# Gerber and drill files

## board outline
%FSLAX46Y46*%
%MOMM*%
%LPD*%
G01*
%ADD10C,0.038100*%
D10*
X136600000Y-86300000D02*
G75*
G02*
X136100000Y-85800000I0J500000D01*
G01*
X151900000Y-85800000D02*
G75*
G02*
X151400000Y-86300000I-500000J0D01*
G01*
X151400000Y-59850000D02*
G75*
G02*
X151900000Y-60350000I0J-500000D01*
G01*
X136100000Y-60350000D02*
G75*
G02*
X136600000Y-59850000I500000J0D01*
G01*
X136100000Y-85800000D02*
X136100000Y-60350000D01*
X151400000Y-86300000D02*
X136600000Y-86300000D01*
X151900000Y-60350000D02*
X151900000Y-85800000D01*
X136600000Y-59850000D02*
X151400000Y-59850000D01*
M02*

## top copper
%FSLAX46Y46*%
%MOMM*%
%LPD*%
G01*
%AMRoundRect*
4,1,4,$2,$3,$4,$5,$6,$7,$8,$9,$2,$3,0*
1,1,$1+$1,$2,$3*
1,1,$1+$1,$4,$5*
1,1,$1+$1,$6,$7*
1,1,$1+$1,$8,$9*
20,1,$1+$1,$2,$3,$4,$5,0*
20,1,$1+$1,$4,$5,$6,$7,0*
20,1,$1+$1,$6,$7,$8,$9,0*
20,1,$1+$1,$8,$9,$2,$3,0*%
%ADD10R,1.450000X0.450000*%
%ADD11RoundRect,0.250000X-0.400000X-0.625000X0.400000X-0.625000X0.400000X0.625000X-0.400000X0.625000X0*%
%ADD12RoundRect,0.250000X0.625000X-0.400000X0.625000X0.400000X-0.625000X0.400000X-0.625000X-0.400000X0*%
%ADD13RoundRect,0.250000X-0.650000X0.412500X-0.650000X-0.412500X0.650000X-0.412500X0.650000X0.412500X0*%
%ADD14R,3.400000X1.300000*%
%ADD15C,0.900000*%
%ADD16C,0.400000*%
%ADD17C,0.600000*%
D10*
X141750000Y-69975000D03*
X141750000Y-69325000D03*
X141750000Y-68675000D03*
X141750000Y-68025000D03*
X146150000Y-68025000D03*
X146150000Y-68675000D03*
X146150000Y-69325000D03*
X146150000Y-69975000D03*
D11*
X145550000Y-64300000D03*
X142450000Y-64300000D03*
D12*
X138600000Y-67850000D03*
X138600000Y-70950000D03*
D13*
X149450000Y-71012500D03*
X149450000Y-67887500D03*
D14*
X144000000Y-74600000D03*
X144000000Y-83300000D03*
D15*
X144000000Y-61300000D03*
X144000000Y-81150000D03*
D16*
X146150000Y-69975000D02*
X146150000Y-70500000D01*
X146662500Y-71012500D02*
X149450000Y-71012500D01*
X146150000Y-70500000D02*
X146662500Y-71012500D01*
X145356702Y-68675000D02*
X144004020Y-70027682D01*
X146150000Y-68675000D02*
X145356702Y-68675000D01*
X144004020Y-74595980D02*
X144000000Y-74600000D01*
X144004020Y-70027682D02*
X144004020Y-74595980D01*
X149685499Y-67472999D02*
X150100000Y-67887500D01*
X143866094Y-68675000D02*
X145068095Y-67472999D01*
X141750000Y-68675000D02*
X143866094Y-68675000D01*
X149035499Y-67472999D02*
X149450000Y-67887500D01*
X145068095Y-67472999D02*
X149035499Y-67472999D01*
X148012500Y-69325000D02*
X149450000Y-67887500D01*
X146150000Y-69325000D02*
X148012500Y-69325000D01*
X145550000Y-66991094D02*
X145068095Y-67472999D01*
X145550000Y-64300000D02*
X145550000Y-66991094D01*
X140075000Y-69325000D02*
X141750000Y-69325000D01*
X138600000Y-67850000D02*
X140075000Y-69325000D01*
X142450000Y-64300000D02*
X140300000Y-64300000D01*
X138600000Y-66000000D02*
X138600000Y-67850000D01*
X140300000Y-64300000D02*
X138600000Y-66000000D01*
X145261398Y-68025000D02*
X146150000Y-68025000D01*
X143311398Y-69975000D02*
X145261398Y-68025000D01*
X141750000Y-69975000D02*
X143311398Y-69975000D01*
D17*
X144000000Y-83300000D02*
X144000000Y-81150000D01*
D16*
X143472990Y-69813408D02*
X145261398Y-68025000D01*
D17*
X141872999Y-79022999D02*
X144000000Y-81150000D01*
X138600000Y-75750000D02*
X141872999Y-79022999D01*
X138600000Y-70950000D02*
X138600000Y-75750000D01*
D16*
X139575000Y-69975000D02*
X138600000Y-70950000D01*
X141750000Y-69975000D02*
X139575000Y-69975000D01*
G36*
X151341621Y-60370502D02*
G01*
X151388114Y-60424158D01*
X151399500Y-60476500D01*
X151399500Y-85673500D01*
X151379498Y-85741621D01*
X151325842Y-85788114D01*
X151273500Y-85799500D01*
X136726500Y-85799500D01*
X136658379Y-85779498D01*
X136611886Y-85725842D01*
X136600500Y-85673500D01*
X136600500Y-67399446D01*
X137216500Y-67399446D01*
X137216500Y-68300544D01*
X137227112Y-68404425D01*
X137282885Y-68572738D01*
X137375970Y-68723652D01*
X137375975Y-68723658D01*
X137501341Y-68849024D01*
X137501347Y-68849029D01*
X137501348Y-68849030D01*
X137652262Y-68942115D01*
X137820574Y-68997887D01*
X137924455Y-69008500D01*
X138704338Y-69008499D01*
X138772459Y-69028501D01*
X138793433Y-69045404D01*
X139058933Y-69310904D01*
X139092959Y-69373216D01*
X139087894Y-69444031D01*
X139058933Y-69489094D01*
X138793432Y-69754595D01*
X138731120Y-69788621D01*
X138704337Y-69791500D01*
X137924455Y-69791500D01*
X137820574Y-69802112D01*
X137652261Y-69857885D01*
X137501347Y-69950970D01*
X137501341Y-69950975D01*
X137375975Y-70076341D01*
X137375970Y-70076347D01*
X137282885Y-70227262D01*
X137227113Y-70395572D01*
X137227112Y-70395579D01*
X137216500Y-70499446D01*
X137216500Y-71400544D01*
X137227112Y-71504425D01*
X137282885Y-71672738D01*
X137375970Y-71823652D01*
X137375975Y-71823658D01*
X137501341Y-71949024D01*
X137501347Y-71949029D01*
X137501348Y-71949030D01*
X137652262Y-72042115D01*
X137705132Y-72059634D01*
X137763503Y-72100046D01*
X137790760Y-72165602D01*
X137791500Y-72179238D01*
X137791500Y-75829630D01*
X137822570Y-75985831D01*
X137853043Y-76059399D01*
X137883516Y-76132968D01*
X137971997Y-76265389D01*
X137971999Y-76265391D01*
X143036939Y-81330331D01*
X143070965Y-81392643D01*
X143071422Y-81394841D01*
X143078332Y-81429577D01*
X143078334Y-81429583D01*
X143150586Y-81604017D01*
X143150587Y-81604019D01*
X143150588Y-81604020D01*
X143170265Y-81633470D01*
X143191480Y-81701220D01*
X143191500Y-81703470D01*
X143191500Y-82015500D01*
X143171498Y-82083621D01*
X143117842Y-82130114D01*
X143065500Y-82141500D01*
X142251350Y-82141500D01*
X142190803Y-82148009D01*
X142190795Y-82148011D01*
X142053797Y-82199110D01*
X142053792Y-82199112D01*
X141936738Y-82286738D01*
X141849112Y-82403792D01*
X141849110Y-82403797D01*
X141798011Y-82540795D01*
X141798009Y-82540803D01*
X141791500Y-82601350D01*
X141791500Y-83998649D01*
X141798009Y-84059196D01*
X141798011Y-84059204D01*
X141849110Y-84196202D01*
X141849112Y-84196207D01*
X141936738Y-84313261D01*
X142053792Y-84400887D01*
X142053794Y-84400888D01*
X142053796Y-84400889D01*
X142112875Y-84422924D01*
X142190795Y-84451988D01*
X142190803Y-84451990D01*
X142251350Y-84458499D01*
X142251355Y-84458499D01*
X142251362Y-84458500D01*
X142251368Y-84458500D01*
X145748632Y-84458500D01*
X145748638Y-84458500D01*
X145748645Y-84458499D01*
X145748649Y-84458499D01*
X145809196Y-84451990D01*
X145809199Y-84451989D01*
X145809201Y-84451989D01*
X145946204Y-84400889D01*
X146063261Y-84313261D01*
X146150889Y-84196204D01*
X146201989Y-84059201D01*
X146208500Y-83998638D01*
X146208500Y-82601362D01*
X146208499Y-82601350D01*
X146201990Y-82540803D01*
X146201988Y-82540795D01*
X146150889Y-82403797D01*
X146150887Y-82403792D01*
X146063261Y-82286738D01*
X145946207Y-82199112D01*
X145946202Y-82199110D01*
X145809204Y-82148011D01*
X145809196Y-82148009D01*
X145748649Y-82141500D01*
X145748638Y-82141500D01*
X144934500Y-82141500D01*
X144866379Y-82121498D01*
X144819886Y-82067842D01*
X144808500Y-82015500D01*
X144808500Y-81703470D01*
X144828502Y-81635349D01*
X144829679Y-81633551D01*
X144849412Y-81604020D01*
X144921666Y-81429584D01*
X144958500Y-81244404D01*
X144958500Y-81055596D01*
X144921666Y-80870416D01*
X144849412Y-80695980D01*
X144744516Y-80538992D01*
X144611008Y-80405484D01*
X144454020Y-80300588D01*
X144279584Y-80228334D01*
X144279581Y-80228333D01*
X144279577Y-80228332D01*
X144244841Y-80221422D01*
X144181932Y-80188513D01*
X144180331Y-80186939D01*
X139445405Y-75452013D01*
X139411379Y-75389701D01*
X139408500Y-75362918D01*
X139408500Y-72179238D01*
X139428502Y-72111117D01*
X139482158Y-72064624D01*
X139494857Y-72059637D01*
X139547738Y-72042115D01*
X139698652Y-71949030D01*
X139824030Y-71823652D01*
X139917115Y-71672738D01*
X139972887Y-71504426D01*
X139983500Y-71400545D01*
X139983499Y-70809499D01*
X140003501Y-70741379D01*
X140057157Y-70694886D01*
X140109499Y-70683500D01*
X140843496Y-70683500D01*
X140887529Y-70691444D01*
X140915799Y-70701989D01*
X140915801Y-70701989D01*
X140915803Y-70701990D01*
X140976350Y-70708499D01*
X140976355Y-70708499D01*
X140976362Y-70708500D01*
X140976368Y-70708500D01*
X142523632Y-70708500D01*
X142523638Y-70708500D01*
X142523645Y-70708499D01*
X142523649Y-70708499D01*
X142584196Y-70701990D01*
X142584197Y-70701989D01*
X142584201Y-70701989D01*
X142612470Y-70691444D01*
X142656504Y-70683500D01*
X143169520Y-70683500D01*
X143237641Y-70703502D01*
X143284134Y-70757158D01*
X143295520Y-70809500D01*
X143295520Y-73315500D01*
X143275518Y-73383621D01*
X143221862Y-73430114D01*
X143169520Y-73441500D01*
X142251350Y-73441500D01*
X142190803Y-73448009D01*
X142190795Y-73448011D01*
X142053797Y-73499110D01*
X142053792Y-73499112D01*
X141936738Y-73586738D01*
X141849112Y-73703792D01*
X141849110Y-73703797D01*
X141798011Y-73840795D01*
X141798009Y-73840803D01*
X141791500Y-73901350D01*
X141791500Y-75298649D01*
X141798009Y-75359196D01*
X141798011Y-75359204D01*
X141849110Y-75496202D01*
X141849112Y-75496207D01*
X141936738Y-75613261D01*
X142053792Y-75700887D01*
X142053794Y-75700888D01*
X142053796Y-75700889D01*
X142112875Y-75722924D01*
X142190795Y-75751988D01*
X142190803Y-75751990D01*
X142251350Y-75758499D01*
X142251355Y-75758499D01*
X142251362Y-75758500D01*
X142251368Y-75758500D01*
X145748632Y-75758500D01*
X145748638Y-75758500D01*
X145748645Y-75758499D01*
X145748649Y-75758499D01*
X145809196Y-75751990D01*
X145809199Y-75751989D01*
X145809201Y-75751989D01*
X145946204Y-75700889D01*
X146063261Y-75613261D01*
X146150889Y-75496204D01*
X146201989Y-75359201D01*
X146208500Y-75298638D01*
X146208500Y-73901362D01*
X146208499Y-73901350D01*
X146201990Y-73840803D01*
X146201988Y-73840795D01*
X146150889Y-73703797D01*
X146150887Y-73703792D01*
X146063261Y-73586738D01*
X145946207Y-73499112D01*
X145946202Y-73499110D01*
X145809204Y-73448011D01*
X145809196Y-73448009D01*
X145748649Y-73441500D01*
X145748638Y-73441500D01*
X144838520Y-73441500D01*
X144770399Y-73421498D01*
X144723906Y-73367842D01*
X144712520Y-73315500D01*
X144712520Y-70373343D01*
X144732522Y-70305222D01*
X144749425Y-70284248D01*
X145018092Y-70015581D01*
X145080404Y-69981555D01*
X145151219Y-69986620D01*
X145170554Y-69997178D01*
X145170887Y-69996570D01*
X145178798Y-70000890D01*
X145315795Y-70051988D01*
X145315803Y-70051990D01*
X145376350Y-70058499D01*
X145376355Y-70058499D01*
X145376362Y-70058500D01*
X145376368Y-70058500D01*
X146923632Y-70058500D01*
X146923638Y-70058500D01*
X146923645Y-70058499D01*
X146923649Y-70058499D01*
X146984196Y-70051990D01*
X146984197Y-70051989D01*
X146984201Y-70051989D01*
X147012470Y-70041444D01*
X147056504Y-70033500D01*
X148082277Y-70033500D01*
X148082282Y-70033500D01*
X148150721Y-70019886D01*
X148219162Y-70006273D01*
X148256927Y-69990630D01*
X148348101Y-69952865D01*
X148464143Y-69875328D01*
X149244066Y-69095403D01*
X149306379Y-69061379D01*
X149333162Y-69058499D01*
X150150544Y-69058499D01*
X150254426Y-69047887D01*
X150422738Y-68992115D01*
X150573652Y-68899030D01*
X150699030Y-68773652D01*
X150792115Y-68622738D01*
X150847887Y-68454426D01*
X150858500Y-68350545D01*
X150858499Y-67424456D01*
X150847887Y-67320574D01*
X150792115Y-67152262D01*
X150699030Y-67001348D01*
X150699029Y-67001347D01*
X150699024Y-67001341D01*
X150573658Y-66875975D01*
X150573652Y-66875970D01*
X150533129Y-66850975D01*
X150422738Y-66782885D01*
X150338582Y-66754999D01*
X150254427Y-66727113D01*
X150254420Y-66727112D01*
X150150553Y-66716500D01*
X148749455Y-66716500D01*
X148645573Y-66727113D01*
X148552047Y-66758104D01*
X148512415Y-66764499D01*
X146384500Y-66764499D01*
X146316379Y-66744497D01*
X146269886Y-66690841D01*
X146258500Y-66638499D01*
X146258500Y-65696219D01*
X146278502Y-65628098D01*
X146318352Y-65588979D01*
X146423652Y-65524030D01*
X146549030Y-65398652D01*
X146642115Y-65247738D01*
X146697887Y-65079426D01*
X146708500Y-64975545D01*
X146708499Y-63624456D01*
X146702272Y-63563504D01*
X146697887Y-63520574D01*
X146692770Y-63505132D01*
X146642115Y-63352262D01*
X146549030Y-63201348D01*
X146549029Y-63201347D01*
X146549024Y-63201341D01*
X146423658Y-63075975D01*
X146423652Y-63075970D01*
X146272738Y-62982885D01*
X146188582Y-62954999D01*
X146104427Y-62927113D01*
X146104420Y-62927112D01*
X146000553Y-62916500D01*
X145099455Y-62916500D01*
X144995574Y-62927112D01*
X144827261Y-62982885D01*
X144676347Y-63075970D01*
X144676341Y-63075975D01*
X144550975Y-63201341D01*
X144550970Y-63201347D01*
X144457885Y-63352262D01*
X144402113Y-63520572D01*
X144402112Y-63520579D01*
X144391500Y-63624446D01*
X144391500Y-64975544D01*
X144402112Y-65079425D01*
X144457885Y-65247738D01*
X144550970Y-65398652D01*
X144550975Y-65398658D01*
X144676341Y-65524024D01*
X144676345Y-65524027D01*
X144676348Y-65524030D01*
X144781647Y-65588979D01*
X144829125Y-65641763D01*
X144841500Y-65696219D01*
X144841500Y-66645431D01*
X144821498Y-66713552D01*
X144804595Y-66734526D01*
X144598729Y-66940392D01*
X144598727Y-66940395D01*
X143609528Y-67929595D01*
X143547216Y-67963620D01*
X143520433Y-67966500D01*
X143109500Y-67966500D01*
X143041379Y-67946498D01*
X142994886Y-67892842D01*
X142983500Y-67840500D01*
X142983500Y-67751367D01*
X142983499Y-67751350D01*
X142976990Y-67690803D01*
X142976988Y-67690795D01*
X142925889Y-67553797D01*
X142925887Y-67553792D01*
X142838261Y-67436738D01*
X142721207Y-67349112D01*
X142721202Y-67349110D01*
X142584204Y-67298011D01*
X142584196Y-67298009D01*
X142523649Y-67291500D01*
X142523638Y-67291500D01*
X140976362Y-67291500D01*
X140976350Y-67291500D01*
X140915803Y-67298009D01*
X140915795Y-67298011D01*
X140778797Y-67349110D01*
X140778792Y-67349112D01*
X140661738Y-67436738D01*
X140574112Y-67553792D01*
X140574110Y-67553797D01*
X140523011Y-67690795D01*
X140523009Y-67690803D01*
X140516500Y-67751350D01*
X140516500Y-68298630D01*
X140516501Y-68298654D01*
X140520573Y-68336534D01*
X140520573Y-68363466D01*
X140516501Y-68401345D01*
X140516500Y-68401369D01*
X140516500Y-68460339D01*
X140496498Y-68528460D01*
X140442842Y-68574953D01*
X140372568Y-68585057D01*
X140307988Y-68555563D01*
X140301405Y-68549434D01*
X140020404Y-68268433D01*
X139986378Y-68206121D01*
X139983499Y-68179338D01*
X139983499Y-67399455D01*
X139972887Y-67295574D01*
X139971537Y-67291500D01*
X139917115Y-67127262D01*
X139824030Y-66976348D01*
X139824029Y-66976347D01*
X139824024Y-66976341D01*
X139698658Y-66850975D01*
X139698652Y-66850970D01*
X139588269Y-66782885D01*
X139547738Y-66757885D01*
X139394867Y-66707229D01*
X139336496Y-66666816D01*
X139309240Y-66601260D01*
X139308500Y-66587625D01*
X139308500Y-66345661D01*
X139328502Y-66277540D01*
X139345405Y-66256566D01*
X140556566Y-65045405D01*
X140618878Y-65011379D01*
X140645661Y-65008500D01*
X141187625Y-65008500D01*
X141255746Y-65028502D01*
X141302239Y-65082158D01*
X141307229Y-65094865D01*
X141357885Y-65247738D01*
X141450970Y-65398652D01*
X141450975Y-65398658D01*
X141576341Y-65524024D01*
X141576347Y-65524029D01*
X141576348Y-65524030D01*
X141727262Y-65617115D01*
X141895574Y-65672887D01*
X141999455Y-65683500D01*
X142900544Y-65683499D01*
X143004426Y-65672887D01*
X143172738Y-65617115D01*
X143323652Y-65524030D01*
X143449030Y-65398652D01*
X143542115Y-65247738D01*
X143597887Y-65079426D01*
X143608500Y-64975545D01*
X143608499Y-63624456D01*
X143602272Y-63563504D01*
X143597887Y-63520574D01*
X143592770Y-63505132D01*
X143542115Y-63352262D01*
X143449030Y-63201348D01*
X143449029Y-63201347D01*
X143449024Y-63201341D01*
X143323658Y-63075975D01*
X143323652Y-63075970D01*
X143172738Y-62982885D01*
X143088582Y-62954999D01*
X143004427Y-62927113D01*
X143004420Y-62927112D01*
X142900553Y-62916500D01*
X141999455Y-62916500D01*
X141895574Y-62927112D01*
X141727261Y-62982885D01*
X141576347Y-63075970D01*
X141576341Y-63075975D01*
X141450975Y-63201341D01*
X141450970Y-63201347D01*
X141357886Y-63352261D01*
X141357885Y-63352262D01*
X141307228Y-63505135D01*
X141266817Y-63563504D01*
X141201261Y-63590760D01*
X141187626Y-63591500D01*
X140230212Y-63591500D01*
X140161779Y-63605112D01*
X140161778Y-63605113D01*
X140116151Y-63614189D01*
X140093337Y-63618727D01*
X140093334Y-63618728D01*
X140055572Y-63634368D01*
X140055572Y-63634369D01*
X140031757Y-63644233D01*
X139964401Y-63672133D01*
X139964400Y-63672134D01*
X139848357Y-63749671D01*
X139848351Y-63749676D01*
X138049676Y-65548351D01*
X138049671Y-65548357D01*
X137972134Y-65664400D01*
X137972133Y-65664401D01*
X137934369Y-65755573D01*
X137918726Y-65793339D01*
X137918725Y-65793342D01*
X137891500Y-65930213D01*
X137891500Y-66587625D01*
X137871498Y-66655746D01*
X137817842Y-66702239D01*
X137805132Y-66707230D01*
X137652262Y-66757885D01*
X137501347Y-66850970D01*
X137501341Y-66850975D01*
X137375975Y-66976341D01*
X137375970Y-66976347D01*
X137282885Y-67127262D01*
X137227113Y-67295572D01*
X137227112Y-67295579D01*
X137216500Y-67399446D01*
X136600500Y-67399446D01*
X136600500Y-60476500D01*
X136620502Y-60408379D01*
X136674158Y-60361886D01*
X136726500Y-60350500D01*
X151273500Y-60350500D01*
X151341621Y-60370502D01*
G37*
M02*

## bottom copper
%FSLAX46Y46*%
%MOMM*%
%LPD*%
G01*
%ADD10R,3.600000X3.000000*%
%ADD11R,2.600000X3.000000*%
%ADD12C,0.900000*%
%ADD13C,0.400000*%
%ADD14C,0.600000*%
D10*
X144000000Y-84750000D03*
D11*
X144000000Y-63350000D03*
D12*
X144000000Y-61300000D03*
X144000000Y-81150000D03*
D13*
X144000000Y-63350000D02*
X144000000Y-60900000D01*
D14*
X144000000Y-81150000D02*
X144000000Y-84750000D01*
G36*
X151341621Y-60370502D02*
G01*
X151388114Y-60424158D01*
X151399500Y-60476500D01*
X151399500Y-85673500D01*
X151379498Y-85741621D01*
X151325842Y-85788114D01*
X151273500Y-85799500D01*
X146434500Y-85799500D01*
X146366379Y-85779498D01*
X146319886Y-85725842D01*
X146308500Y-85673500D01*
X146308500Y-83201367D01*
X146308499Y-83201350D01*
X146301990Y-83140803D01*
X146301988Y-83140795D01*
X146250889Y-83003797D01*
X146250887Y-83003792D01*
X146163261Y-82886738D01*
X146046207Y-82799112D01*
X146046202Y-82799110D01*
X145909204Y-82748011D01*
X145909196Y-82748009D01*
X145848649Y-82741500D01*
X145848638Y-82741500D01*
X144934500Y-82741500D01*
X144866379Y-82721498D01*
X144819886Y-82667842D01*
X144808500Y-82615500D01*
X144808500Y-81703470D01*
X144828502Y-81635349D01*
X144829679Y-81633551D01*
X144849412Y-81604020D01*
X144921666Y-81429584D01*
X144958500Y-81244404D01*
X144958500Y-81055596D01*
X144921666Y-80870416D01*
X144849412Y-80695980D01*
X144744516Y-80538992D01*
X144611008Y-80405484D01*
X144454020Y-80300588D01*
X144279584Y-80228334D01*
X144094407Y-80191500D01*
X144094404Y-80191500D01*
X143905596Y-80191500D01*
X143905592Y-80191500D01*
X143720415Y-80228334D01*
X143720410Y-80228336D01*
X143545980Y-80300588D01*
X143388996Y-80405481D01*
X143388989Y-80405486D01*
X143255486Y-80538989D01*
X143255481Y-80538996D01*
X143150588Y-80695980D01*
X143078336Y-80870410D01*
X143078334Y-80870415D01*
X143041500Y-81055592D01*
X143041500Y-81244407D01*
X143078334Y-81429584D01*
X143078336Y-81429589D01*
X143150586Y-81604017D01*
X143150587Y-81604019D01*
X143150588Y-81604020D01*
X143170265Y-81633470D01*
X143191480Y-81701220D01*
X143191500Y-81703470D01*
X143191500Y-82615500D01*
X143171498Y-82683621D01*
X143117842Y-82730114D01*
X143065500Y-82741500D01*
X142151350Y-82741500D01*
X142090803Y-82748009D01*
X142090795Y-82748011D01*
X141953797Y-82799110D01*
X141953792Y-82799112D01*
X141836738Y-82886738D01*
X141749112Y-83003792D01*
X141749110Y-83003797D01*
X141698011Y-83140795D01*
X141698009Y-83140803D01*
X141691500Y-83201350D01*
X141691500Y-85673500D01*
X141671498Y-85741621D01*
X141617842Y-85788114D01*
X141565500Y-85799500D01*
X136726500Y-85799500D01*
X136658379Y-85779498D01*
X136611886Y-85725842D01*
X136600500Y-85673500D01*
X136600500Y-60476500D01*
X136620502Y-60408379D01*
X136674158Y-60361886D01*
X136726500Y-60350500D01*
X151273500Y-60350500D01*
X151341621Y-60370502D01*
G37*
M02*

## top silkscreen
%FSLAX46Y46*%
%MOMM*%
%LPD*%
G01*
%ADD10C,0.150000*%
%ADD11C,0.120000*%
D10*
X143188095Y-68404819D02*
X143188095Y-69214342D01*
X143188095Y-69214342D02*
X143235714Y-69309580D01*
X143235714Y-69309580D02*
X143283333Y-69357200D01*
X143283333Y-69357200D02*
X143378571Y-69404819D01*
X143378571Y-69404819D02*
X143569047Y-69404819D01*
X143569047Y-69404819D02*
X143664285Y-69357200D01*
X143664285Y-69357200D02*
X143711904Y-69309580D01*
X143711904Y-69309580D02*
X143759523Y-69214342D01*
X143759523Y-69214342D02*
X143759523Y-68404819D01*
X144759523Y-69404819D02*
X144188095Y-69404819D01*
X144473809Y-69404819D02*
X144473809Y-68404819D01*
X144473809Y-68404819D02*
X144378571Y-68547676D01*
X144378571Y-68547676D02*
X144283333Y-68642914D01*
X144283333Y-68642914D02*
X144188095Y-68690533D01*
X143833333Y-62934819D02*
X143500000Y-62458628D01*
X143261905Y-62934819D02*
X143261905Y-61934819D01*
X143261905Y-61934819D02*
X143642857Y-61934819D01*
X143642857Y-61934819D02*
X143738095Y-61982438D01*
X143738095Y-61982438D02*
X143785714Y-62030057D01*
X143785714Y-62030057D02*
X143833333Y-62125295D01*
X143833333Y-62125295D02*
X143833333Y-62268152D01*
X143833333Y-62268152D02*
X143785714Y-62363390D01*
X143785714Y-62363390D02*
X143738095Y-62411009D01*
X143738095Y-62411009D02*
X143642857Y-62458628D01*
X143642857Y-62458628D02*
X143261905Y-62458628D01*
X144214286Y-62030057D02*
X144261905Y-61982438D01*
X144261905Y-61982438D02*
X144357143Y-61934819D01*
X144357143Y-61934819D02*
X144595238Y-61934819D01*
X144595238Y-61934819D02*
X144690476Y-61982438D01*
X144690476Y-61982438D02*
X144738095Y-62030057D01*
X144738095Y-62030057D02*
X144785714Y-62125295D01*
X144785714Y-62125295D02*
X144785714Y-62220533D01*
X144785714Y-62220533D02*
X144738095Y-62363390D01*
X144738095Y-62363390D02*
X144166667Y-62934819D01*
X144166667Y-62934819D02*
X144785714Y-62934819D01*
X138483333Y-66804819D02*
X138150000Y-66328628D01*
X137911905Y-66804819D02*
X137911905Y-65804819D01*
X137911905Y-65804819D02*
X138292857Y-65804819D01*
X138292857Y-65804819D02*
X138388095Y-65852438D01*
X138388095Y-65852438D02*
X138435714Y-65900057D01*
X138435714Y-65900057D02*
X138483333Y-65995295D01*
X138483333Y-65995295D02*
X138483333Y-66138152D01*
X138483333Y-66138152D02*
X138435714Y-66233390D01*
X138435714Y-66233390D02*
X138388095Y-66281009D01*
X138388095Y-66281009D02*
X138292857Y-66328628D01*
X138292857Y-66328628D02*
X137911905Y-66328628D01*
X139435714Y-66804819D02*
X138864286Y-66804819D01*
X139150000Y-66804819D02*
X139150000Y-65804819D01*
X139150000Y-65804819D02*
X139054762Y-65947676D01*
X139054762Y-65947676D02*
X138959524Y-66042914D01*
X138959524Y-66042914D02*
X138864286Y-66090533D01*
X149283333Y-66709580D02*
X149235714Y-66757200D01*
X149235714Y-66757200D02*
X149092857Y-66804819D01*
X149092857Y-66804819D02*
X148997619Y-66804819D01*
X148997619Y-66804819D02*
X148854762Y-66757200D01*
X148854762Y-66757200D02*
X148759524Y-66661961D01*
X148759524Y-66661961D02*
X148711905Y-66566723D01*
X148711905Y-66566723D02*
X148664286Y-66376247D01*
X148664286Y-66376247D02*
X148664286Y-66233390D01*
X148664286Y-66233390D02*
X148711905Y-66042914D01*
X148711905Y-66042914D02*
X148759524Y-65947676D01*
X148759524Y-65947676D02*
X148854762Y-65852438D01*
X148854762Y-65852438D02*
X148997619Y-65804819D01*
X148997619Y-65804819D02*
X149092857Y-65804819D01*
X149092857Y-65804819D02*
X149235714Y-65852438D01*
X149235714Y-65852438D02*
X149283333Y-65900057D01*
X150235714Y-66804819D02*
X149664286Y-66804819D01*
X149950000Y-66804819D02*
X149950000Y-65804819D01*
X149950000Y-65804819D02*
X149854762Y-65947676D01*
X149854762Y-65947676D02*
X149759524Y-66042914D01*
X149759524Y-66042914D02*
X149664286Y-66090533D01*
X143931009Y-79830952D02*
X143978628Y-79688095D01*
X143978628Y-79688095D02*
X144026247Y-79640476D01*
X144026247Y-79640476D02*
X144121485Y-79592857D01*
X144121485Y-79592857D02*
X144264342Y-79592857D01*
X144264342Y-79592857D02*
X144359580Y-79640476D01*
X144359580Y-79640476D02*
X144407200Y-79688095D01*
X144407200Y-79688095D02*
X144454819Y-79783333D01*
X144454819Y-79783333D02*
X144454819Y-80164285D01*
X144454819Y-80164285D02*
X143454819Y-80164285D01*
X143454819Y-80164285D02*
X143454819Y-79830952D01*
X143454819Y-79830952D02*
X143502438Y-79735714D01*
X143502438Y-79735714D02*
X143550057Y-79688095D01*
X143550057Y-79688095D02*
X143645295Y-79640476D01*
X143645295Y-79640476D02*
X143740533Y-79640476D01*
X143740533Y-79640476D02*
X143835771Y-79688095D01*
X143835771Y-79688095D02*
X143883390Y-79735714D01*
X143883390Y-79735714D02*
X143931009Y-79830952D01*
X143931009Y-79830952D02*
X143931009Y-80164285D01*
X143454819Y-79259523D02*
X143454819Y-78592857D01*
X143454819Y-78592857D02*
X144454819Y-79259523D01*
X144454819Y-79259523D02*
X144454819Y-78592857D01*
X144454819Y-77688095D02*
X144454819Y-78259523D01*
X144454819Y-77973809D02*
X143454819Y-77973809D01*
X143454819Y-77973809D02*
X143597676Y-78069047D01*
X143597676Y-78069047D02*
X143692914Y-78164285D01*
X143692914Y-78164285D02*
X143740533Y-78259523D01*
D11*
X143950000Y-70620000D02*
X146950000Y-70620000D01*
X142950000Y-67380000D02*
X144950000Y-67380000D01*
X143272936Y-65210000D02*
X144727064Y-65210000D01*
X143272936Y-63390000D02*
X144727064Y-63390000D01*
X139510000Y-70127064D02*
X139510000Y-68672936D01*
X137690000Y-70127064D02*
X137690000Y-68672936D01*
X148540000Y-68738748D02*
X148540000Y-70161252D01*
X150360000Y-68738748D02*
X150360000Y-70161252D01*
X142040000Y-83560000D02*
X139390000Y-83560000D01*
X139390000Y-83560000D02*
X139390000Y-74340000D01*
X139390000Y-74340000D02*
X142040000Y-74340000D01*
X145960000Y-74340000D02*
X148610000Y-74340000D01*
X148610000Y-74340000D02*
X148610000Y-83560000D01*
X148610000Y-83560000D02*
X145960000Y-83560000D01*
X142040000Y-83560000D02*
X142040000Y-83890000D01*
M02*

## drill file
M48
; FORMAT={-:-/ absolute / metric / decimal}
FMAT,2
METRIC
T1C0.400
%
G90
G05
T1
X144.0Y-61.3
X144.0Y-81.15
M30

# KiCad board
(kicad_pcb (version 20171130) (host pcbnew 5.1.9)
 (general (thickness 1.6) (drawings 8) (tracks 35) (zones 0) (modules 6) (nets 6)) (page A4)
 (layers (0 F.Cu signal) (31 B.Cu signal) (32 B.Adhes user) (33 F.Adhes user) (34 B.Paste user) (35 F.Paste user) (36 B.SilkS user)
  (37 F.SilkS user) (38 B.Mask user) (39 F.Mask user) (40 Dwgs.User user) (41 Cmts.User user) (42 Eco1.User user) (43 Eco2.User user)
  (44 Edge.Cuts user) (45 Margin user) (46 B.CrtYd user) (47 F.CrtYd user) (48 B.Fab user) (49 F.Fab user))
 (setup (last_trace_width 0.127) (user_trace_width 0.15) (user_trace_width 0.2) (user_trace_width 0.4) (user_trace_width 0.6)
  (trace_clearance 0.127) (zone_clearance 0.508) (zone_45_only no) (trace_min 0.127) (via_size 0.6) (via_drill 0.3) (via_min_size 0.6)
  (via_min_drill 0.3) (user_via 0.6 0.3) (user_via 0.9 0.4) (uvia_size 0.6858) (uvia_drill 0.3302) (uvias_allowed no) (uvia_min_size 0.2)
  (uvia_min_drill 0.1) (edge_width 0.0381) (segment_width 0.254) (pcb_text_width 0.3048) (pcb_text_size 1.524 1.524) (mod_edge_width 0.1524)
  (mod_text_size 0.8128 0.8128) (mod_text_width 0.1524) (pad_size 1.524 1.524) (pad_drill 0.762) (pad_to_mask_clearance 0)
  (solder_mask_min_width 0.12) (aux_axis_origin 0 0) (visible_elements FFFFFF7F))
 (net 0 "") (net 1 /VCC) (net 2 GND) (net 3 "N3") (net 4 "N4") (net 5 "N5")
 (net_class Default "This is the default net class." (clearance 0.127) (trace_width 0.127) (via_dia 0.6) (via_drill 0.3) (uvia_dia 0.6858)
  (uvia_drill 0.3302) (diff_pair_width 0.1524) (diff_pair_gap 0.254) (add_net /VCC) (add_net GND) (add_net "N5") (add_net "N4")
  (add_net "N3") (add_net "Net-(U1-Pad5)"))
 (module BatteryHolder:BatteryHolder (layer B.Cu) (at 144 71.85 180)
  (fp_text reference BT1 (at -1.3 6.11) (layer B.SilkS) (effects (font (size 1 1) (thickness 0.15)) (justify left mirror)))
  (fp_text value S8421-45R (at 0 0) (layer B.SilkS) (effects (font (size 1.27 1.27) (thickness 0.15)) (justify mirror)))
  (pad 2 smd rect (at 0 -12.9 180) (size 3.6 3) (layers B.Cu B.Paste B.Mask) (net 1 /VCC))
  (pad 1 smd rect (at 0 8.5 180) (size 2.6 3) (layers B.Cu B.Paste B.Mask) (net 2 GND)))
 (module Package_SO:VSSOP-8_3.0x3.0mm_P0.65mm (layer F.Cu) (at 143.95 69 180)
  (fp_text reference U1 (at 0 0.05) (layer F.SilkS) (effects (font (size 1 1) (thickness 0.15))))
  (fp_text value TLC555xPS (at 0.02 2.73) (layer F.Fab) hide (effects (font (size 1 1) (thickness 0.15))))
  (fp_line (start 0 -1.62) (end -3 -1.62) (layer F.SilkS) (width 0.12))
  (fp_line (start 1 1.62) (end -1 1.62) (layer F.SilkS) (width 0.12))
  (pad 8 smd rect (at 2.2 -0.975 90) (size 0.45 1.45) (layers F.Cu F.Paste F.Mask) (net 1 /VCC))
  (pad 7 smd rect (at 2.2 -0.325 90) (size 0.45 1.45) (layers F.Cu F.Paste F.Mask) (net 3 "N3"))
  (pad 6 smd rect (at 2.2 0.325 90) (size 0.45 1.45) (layers F.Cu F.Paste F.Mask) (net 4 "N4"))
  (pad 5 smd rect (at 2.2 0.975 90) (size 0.45 1.45) (layers F.Cu F.Paste F.Mask))
  (pad 4 smd rect (at -2.2 0.975 90) (size 0.45 1.45) (layers F.Cu F.Paste F.Mask) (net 1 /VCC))
  (pad 3 smd rect (at -2.2 0.325 90) (size 0.45 1.45) (layers F.Cu F.Paste F.Mask) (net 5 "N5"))
  (pad 2 smd rect (at -2.2 -0.325 90) (size 0.45 1.45) (layers F.Cu F.Paste F.Mask) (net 4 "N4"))
  (pad 1 smd rect (at -2.2 -0.975 90) (size 0.45 1.45) (layers F.Cu F.Paste F.Mask) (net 2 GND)))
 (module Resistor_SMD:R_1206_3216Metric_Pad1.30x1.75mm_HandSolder (layer F.Cu) (at 144 64.3)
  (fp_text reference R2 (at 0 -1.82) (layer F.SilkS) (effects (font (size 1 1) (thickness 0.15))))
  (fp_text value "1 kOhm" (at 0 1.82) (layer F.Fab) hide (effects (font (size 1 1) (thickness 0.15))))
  (fp_line (start -0.727064 0.91) (end 0.727064 0.91) (layer F.SilkS) (width 0.12))
  (fp_line (start -0.727064 -0.91) (end 0.727064 -0.91) (layer F.SilkS) (width 0.12))
  (pad 2 smd roundrect (at 1.55 0) (size 1.3 1.75) (layers F.Cu F.Paste F.Mask) (roundrect_rratio 0.192308) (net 4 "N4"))
  (pad 1 smd roundrect (at -1.55 0) (size 1.3 1.75) (layers F.Cu F.Paste F.Mask) (roundrect_rratio 0.192308) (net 3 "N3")))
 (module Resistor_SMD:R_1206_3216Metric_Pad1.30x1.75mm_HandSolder (layer F.Cu) (at 138.6 69.4 90)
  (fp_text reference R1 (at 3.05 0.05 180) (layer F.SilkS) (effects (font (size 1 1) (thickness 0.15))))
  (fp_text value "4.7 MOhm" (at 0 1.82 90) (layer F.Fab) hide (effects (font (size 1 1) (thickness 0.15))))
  (fp_line (start -0.727064 0.91) (end 0.727064 0.91) (layer F.SilkS) (width 0.12))
  (fp_line (start -0.727064 -0.91) (end 0.727064 -0.91) (layer F.SilkS) (width 0.12))
  (pad 2 smd roundrect (at 1.55 0 90) (size 1.3 1.75) (layers F.Cu F.Paste F.Mask) (roundrect_rratio 0.192308) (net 3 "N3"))
  (pad 1 smd roundrect (at -1.55 0 90) (size 1.3 1.75) (layers F.Cu F.Paste F.Mask) (roundrect_rratio 0.192308) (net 1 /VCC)))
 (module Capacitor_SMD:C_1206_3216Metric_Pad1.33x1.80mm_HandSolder (layer F.Cu) (at 149.45 69.45 270)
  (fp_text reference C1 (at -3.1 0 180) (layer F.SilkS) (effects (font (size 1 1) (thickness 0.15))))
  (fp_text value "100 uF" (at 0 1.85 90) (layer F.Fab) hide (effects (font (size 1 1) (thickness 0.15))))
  (fp_line (start -0.711252 0.91) (end 0.711252 0.91) (layer F.SilkS) (width 0.12))
  (fp_line (start -0.711252 -0.91) (end 0.711252 -0.91) (layer F.SilkS) (width 0.12))
  (pad 2 smd roundrect (at 1.5625 0 270) (size 1.325 1.8) (layers F.Cu F.Paste F.Mask) (roundrect_rratio 0.188679) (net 2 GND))
  (pad 1 smd roundrect (at -1.5625 0 270) (size 1.325 1.8) (layers F.Cu F.Paste F.Mask) (roundrect_rratio 0.188679) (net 4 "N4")))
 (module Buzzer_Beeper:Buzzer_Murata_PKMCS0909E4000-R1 (layer F.Cu) (at 144 78.95 90)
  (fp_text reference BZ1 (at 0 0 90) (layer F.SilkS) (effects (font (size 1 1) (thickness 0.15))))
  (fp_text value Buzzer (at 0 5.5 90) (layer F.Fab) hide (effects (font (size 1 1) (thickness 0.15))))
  (fp_line (start -4.61 -1.96) (end -4.61 -4.61) (layer F.SilkS) (width 0.12))
  (fp_line (start -4.61 -4.61) (end 4.61 -4.61) (layer F.SilkS) (width 0.12))
  (fp_line (start 4.61 -4.61) (end 4.61 -1.96) (layer F.SilkS) (width 0.12))
  (fp_line (start 4.61 1.96) (end 4.61 4.61) (layer F.SilkS) (width 0.12))
  (fp_line (start 4.61 4.61) (end -4.61 4.61) (layer F.SilkS) (width 0.12))
  (fp_line (start -4.61 4.61) (end -4.61 1.96) (layer F.SilkS) (width 0.12))
  (fp_line (start -4.61 -1.96) (end -4.94 -1.96) (layer F.SilkS) (width 0.12))
  (pad 2 smd rect (at 4.35 0 90) (size 1.3 3.4) (layers F.Cu F.Paste F.Mask) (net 5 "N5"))
  (pad 1 smd rect (at -4.35 0 90) (size 1.3 3.4) (layers F.Cu F.Paste F.Mask) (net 1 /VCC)))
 (gr_arc (start 136.6 85.8) (end 136.1 85.8) (angle -90) (layer Edge.Cuts) (width 0.0381))
 (gr_arc (start 151.4 85.8) (end 151.4 86.3) (angle -90) (layer Edge.Cuts) (width 0.0381))
 (gr_arc (start 151.4 60.35) (end 151.9 60.35) (angle -90) (layer Edge.Cuts) (width 0.0381))
 (gr_arc (start 136.6 60.35) (end 136.6 59.85) (angle -90) (layer Edge.Cuts) (width 0.0381))
 (gr_line (start 136.1 85.8) (end 136.1 60.35) (layer Edge.Cuts) (width 0.0381))
 (gr_line (start 151.4 86.3) (end 136.6 86.3) (layer Edge.Cuts) (width 0.0381))
 (gr_line (start 151.9 60.35) (end 151.9 85.8) (layer Edge.Cuts) (width 0.0381))
 (gr_line (start 136.6 59.85) (end 151.4 59.85) (layer Edge.Cuts) (width 0.0381))
 (via (at 144 61.3) (size 0.9) (drill 0.4) (layers F.Cu B.Cu) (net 2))
 (segment (start 144 63.35) (end 144 60.9) (width 0.4) (layer B.Cu) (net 2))
 (segment (start 146.15 69.975) (end 146.15 70.5) (width 0.4) (layer F.Cu) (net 2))
 (segment (start 146.6625 71.0125) (end 149.45 71.0125) (width 0.4) (layer F.Cu) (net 2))
 (segment (start 146.15 70.5) (end 146.6625 71.0125) (width 0.4) (layer F.Cu) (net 2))
 (segment (start 145.356702 68.675) (end 144.00402 70.027682) (width 0.4) (layer F.Cu) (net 5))
 (segment (start 146.15 68.675) (end 145.356702 68.675) (width 0.4) (layer F.Cu) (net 5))
 (segment (start 144.00402 74.59598) (end 144 74.6) (width 0.4) (layer F.Cu) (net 5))
 (segment (start 144.00402 70.027682) (end 144.00402 74.59598) (width 0.4) (layer F.Cu) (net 5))
 (segment (start 149.685499 67.472999) (end 150.1 67.8875) (width 0.4) (layer F.Cu) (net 4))
 (segment (start 143.866094 68.675) (end 145.068095 67.472999) (width 0.4) (layer F.Cu) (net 4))
 (segment (start 141.75 68.675) (end 143.866094 68.675) (width 0.4) (layer F.Cu) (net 4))
 (segment (start 149.035499 67.472999) (end 149.45 67.8875) (width 0.4) (layer F.Cu) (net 4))
 (segment (start 145.068095 67.472999) (end 149.035499 67.472999) (width 0.4) (layer F.Cu) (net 4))
 (segment (start 148.0125 69.325) (end 149.45 67.8875) (width 0.4) (layer F.Cu) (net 4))
 (segment (start 146.15 69.325) (end 148.0125 69.325) (width 0.4) (layer F.Cu) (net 4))
 (segment (start 145.55 66.991094) (end 145.068095 67.472999) (width 0.4) (layer F.Cu) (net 4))
 (segment (start 145.55 64.3) (end 145.55 66.991094) (width 0.4) (layer F.Cu) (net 4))
 (segment (start 140.075 69.325) (end 141.75 69.325) (width 0.4) (layer F.Cu) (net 3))
 (segment (start 138.6 67.85) (end 140.075 69.325) (width 0.4) (layer F.Cu) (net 3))
 (segment (start 142.45 64.3) (end 140.3 64.3) (width 0.4) (layer F.Cu) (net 3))
 (segment (start 138.6 66) (end 138.6 67.85) (width 0.4) (layer F.Cu) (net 3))
 (segment (start 140.3 64.3) (end 138.6 66) (width 0.4) (layer F.Cu) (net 3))
 (segment (start 145.261398 68.025) (end 146.15 68.025) (width 0.4) (layer F.Cu) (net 1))
 (segment (start 143.311398 69.975) (end 145.261398 68.025) (width 0.4) (layer F.Cu) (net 1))
 (segment (start 141.75 69.975) (end 143.311398 69.975) (width 0.4) (layer F.Cu) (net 1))
 (via (at 144 81.15) (size 0.9) (drill 0.4) (layers F.Cu B.Cu) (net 1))
 (segment (start 144 83.3) (end 144 81.15) (width 0.6) (layer F.Cu) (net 1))
 (segment (start 144 81.15) (end 144 84.75) (width 0.6) (layer B.Cu) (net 1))
 (segment (start 143.47299 69.813408) (end 145.261398 68.025) (width 0.4) (layer F.Cu) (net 1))
 (segment (start 141.872999 79.022999) (end 144 81.15) (width 0.6) (layer F.Cu) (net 1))
 (segment (start 138.6 75.75) (end 141.872999 79.022999) (width 0.6) (layer F.Cu) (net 1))
 (segment (start 138.6 70.95) (end 138.6 75.75) (width 0.6) (layer F.Cu) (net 1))
 (segment (start 139.575 69.975) (end 138.6 70.95) (width 0.4) (layer F.Cu) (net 1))
 (segment (start 141.75 69.975) (end 139.575 69.975) (width 0.4) (layer F.Cu) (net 1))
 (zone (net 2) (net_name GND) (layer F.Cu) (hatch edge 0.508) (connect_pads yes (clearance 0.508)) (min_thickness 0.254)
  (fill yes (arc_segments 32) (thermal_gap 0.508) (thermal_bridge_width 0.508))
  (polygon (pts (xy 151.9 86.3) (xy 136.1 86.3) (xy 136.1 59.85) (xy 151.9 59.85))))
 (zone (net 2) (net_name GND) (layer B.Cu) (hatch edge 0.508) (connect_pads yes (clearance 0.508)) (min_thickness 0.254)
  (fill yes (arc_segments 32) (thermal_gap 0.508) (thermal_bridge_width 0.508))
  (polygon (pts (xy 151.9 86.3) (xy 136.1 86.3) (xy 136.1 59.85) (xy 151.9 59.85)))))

